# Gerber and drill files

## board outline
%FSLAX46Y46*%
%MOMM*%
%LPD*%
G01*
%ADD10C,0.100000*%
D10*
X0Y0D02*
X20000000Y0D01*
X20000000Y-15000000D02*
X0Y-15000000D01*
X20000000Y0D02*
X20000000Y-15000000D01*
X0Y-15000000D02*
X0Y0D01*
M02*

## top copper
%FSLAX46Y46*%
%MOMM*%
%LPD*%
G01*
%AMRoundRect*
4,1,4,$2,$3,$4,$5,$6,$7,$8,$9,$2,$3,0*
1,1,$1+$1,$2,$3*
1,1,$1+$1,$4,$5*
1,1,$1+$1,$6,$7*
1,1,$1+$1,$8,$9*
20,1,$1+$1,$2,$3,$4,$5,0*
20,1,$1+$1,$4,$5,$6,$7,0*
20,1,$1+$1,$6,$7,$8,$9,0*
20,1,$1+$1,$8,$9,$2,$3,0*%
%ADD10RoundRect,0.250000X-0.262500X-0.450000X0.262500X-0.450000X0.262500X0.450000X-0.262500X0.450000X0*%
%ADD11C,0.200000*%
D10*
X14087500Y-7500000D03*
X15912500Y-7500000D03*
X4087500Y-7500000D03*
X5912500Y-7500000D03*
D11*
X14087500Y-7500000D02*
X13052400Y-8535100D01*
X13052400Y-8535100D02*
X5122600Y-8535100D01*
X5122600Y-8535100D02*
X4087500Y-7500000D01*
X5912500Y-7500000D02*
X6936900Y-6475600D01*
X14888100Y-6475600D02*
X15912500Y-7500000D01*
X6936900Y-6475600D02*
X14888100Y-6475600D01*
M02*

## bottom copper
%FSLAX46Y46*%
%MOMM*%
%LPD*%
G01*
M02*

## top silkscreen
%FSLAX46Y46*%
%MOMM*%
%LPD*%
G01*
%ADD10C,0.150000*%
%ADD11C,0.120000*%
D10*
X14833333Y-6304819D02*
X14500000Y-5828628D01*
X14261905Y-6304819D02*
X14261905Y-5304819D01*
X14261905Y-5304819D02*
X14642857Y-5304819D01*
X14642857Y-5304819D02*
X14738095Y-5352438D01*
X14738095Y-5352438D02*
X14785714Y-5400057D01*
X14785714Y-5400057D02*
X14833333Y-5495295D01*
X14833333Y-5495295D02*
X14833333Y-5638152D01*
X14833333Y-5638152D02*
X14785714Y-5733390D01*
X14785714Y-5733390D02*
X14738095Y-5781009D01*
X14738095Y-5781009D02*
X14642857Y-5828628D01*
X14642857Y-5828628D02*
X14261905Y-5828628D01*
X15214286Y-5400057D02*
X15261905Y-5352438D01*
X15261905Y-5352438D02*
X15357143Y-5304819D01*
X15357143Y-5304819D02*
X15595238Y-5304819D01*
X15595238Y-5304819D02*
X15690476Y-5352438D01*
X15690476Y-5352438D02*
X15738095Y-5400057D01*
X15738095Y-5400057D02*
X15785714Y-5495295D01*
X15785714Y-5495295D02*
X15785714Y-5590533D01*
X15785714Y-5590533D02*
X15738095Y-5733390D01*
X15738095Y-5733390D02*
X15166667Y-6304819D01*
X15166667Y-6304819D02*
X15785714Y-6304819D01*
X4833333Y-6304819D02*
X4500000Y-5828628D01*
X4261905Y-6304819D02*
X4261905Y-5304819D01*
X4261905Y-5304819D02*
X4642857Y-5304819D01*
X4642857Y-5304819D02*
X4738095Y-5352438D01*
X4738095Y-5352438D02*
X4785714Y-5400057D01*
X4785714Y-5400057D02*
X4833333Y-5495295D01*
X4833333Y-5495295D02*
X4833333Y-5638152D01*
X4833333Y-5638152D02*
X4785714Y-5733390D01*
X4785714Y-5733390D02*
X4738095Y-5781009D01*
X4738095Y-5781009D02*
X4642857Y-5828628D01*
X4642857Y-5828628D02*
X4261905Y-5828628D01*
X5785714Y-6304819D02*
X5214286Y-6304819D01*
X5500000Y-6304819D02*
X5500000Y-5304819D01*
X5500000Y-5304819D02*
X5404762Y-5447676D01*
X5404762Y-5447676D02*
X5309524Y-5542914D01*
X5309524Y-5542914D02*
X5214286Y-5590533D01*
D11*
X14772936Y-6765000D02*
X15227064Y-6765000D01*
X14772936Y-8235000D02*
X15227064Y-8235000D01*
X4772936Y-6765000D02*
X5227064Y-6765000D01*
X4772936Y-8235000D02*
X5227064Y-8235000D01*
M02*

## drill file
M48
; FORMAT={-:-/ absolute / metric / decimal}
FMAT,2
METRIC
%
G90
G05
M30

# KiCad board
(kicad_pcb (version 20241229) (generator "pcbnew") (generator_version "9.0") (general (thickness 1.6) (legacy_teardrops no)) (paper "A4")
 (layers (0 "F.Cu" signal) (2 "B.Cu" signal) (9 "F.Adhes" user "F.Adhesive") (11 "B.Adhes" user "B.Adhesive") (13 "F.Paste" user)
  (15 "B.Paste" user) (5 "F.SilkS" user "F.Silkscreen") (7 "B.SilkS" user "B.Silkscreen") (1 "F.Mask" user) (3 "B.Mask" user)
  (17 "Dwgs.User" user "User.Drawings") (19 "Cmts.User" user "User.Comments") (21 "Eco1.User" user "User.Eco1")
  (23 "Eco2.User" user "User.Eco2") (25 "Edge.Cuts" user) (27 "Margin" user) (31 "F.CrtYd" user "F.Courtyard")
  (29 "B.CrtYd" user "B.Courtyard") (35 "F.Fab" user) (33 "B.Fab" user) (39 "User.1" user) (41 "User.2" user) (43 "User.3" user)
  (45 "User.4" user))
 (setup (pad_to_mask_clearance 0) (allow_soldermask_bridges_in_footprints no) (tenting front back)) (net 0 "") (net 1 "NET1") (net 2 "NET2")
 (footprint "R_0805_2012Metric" (layer "F.Cu") (at 15 7.5)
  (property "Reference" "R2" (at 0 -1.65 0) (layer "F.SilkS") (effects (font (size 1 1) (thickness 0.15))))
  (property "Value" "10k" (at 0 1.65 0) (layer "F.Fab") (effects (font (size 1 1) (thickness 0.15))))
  (fp_line (start -0.227064 -0.735) (end 0.227064 -0.735) (stroke (width 0.12) (type solid)) (layer "F.SilkS"))
  (fp_line (start -0.227064 0.735) (end 0.227064 0.735) (stroke (width 0.12) (type solid)) (layer "F.SilkS"))
  (pad "1" smd roundrect (at -0.9125 0) (size 1.025 1.4) (layers "F.Cu" "F.Mask" "F.Paste") (roundrect_rratio 0.243902) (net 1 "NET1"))
  (pad "2" smd roundrect (at 0.9125 0) (size 1.025 1.4) (layers "F.Cu" "F.Mask" "F.Paste") (roundrect_rratio 0.243902) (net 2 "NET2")))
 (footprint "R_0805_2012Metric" (layer "F.Cu") (at 5 7.5)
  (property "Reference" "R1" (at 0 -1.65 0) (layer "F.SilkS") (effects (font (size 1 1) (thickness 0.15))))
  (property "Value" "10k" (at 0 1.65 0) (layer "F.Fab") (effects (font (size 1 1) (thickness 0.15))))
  (fp_line (start -0.227064 -0.735) (end 0.227064 -0.735) (stroke (width 0.12) (type solid)) (layer "F.SilkS"))
  (fp_line (start -0.227064 0.735) (end 0.227064 0.735) (stroke (width 0.12) (type solid)) (layer "F.SilkS"))
  (pad "1" smd roundrect (at -0.9125 0) (size 1.025 1.4) (layers "F.Cu" "F.Mask" "F.Paste") (roundrect_rratio 0.243902) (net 1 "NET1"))
  (pad "2" smd roundrect (at 0.9125 0) (size 1.025 1.4) (layers "F.Cu" "F.Mask" "F.Paste") (roundrect_rratio 0.243902) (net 2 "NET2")))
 (gr_line (start 0 0) (end 20 0) (stroke (width 0.1) (type default)) (layer "Edge.Cuts"))
 (gr_line (start 20 15) (end 0 15) (stroke (width 0.1) (type default)) (layer "Edge.Cuts"))
 (gr_line (start 20 0) (end 20 15) (stroke (width 0.1) (type default)) (layer "Edge.Cuts"))
 (gr_line (start 0 15) (end 0 0) (stroke (width 0.1) (type default)) (layer "Edge.Cuts"))
 (segment (start 14.0875 7.5) (end 13.0524 8.5351) (width 0.2) (layer "F.Cu") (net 1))
 (segment (start 13.0524 8.5351) (end 5.1226 8.5351) (width 0.2) (layer "F.Cu") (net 1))
 (segment (start 5.1226 8.5351) (end 4.0875 7.5) (width 0.2) (layer "F.Cu") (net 1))
 (segment (start 5.9125 7.5) (end 6.9369 6.4756) (width 0.2) (layer "F.Cu") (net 2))
 (segment (start 14.8881 6.4756) (end 15.9125 7.5) (width 0.2) (layer "F.Cu") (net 2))
 (segment (start 6.9369 6.4756) (end 14.8881 6.4756) (width 0.2) (layer "F.Cu") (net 2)))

